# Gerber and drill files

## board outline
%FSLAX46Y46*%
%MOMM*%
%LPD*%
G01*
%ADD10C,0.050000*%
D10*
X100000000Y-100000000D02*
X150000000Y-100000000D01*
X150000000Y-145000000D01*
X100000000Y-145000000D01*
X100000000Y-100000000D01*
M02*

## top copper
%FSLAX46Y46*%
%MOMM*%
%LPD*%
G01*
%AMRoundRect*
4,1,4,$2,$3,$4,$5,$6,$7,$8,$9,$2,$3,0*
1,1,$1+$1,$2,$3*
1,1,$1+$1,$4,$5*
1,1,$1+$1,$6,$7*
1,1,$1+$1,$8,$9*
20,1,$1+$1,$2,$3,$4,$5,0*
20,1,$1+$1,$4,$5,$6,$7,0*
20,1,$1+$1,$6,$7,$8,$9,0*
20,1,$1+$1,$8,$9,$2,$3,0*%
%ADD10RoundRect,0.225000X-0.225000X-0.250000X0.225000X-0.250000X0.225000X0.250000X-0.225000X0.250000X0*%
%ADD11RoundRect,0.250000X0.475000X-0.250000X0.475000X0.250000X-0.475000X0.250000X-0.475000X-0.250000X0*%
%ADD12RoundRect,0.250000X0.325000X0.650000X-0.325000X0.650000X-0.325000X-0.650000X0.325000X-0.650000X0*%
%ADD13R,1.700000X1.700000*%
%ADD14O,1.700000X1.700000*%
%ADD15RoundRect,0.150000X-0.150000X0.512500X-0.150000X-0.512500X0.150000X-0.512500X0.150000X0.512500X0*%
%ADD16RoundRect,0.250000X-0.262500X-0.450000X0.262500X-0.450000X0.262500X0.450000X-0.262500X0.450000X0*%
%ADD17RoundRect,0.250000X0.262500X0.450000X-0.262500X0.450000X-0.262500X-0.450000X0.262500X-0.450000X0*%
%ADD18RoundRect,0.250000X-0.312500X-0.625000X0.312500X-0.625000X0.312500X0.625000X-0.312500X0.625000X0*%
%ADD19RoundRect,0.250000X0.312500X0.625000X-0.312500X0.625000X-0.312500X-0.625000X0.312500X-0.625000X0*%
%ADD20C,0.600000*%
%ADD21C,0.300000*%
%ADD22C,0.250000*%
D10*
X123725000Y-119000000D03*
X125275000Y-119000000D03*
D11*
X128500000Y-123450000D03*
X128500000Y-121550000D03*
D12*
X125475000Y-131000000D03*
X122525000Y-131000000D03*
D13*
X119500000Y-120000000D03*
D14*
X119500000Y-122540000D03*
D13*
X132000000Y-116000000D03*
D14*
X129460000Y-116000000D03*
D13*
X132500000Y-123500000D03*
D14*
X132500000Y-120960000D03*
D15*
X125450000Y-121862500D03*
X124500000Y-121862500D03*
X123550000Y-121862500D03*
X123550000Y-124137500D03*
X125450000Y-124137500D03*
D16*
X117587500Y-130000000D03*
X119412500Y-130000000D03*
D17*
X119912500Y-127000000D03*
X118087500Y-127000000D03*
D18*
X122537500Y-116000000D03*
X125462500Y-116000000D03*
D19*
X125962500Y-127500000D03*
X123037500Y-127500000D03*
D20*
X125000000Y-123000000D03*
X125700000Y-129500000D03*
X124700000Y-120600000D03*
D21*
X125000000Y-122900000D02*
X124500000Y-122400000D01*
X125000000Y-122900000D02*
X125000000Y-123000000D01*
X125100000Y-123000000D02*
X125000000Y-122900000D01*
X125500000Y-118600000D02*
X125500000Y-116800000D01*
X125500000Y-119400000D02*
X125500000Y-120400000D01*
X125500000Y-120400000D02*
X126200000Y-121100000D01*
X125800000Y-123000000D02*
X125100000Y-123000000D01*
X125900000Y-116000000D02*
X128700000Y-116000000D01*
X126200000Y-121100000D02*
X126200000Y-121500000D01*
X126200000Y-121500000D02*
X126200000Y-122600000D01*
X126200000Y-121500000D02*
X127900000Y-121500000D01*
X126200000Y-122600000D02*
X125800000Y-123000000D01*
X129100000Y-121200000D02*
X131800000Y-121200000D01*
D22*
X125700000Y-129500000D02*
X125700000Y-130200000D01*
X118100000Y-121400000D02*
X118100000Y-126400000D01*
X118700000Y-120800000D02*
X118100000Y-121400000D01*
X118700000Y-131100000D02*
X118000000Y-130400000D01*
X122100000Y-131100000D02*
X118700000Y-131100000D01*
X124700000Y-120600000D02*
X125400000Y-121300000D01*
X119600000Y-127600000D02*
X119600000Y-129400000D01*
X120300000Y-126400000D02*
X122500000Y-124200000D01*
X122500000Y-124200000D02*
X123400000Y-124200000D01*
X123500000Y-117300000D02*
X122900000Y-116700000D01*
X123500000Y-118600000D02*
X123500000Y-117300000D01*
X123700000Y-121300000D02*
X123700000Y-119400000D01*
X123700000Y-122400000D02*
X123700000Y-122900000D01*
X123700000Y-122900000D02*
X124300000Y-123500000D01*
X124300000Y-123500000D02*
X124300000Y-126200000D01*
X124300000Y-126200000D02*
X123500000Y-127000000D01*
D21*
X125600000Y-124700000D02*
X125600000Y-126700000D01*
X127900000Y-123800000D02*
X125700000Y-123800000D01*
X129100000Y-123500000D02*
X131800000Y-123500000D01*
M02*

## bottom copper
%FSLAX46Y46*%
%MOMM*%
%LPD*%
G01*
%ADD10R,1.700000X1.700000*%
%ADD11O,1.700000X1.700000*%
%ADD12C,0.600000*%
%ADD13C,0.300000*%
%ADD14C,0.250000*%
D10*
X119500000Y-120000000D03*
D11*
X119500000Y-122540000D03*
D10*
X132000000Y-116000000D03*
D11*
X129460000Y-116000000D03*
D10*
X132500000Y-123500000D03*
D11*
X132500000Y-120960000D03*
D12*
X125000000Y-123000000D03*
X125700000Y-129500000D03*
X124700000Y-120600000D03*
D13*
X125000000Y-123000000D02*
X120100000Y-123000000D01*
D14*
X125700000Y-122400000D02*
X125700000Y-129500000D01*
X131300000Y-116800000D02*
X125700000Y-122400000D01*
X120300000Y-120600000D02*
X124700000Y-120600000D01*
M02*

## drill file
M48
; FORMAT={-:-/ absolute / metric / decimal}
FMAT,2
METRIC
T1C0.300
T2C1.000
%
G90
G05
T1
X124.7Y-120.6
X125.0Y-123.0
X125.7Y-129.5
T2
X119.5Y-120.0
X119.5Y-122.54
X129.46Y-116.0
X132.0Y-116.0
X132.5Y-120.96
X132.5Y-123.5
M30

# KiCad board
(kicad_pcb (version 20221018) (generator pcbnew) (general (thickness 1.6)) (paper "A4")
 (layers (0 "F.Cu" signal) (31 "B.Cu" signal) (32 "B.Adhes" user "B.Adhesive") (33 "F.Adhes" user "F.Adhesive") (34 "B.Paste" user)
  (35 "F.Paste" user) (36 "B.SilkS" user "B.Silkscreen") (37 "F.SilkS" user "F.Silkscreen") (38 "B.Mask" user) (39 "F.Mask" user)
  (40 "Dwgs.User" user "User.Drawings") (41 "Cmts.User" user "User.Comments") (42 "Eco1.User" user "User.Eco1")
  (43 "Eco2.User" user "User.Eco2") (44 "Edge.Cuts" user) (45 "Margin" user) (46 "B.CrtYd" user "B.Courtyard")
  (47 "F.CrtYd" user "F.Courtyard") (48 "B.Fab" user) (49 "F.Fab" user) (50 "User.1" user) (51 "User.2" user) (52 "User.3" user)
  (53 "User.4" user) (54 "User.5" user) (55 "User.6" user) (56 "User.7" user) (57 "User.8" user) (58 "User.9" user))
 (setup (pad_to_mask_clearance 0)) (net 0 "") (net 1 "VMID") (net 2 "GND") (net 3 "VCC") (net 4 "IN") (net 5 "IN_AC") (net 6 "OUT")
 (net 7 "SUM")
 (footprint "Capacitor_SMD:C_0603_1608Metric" (layer "F.Cu") (at 124.5 119)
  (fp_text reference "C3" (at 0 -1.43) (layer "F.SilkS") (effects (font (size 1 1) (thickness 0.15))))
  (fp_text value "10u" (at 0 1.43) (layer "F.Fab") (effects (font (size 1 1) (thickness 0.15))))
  (pad "1" smd roundrect (at -0.775 0) (size 0.9 0.95) (layers "F.Cu" "F.Paste" "F.Mask") (roundrect_rratio 0.25) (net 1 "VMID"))
  (pad "2" smd roundrect (at 0.775 0) (size 0.9 0.95) (layers "F.Cu" "F.Paste" "F.Mask") (roundrect_rratio 0.25) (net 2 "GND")))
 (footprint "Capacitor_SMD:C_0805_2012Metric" (layer "F.Cu") (at 128.5 122.5 90)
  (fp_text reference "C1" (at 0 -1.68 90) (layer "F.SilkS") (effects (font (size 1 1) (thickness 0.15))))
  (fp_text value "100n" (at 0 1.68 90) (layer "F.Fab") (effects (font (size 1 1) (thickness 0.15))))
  (pad "1" smd roundrect (at -0.95 0 90) (size 1 1.45) (layers "F.Cu" "F.Paste" "F.Mask") (roundrect_rratio 0.25) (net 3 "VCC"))
  (pad "2" smd roundrect (at 0.95 0 90) (size 1 1.45) (layers "F.Cu" "F.Paste" "F.Mask") (roundrect_rratio 0.25) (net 2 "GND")))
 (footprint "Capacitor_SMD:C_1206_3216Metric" (layer "F.Cu") (at 124 131 180)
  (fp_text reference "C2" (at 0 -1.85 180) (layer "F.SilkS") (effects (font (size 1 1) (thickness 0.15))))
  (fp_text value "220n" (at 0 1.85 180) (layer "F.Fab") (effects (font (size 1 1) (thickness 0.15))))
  (pad "1" smd roundrect (at -1.475 0 180) (size 1.15 1.8) (layers "F.Cu" "F.Paste" "F.Mask") (roundrect_rratio 0.217391) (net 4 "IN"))
  (pad "2" smd roundrect (at 1.475 0 180) (size 1.15 1.8) (layers "F.Cu" "F.Paste" "F.Mask") (roundrect_rratio 0.217391) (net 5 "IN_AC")))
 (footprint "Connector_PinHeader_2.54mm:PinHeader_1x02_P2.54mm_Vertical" (layer "F.Cu") (at 119.5 120)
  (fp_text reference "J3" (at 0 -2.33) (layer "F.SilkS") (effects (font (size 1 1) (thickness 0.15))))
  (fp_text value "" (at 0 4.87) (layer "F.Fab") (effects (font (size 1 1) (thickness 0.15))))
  (pad "1" thru_hole rect (at 0 0) (size 1.7 1.7) (drill 1) (layers "*.Cu" "*.Mask") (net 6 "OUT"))
  (pad "2" thru_hole oval (at 0 2.54) (size 1.7 1.7) (drill 1) (layers "*.Cu" "*.Mask") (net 2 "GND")))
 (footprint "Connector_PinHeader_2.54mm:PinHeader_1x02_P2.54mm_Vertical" (layer "F.Cu") (at 132 116 -90)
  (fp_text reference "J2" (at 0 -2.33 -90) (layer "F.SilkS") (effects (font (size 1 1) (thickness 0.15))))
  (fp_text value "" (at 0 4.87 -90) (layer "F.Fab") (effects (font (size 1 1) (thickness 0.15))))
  (pad "1" thru_hole rect (at 0 0 270) (size 1.7 1.7) (drill 1) (layers "*.Cu" "*.Mask") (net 4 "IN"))
  (pad "2" thru_hole oval (at 0 2.54 270) (size 1.7 1.7) (drill 1) (layers "*.Cu" "*.Mask") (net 2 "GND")))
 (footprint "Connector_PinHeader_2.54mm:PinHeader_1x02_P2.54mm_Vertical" (layer "F.Cu") (at 132.5 123.5 180)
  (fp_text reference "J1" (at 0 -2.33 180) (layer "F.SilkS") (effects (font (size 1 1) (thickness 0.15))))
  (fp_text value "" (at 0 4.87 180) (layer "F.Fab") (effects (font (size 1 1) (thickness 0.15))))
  (pad "1" thru_hole rect (at 0 0 180) (size 1.7 1.7) (drill 1) (layers "*.Cu" "*.Mask") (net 3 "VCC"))
  (pad "2" thru_hole oval (at 0 2.54 180) (size 1.7 1.7) (drill 1) (layers "*.Cu" "*.Mask") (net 2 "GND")))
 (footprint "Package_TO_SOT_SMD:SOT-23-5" (layer "F.Cu") (at 124.5 123 -90)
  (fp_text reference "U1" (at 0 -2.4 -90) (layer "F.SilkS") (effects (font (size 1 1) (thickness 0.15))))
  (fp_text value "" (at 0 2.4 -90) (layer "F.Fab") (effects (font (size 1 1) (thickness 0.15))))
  (pad "1" smd roundrect (at -1.1375 -0.95 270) (size 1.325 0.6) (layers "F.Cu" "F.Paste" "F.Mask") (roundrect_rratio 0.25) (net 6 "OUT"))
  (pad "2" smd roundrect (at -1.1375 0 270) (size 1.325 0.6) (layers "F.Cu" "F.Paste" "F.Mask") (roundrect_rratio 0.25) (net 2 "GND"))
  (pad "3" smd roundrect (at -1.1375 0.95 270) (size 1.325 0.6) (layers "F.Cu" "F.Paste" "F.Mask") (roundrect_rratio 0.25) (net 1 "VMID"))
  (pad "4" smd roundrect (at 1.1375 0.95 270) (size 1.325 0.6) (layers "F.Cu" "F.Paste" "F.Mask") (roundrect_rratio 0.25) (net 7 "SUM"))
  (pad "5" smd roundrect (at 1.1375 -0.95 270) (size 1.325 0.6) (layers "F.Cu" "F.Paste" "F.Mask") (roundrect_rratio 0.25) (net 3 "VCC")))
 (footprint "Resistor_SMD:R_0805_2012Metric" (layer "F.Cu") (at 118.5 130)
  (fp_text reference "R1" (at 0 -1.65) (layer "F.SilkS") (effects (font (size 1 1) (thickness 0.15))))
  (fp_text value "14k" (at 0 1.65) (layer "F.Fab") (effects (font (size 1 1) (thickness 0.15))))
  (pad "1" smd roundrect (at -0.9125 0) (size 1.025 1.4) (layers "F.Cu" "F.Paste" "F.Mask") (roundrect_rratio 0.243902) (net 5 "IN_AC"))
  (pad "2" smd roundrect (at 0.9125 0) (size 1.025 1.4) (layers "F.Cu" "F.Paste" "F.Mask") (roundrect_rratio 0.243902) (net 7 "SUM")))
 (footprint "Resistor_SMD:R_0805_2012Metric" (layer "F.Cu") (at 119 127 180)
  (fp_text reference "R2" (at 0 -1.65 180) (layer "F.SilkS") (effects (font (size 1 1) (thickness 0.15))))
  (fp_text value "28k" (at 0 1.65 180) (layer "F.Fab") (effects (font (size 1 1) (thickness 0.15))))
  (pad "1" smd roundrect (at -0.9125 0 180) (size 1.025 1.4) (layers "F.Cu" "F.Paste" "F.Mask") (roundrect_rratio 0.243902) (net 7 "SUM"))
  (pad "2" smd roundrect (at 0.9125 0 180) (size 1.025 1.4) (layers "F.Cu" "F.Paste" "F.Mask") (roundrect_rratio 0.243902) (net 6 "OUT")))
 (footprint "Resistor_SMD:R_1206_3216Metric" (layer "F.Cu") (at 124 116)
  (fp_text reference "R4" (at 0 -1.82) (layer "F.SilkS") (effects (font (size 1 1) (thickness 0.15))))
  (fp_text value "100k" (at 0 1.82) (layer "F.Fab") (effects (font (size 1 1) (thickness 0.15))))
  (pad "1" smd roundrect (at -1.4625 0) (size 1.125 1.75) (layers "F.Cu" "F.Paste" "F.Mask") (roundrect_rratio 0.222222) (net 1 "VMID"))
  (pad "2" smd roundrect (at 1.4625 0) (size 1.125 1.75) (layers "F.Cu" "F.Paste" "F.Mask") (roundrect_rratio 0.222222) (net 2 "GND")))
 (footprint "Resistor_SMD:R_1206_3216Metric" (layer "F.Cu") (at 124.5 127.5 180)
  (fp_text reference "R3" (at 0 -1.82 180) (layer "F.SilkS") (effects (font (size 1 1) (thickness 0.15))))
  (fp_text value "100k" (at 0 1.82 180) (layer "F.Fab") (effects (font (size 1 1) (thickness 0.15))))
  (pad "1" smd roundrect (at -1.4625 0 180) (size 1.125 1.75) (layers "F.Cu" "F.Paste" "F.Mask") (roundrect_rratio 0.222222) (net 3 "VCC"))
  (pad "2" smd roundrect (at 1.4625 0 180) (size 1.125 1.75) (layers "F.Cu" "F.Paste" "F.Mask") (roundrect_rratio 0.222222) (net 1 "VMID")))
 (gr_rect (start 100 100) (end 150 145) (stroke (width 0.05) (type default)) (fill none) (layer "Edge.Cuts"))
 (segment (start 125 122.9) (end 124.5 122.4) (width 0.3) (layer "F.Cu") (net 2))
 (segment (start 125 122.9) (end 125 123) (width 0.3) (layer "F.Cu") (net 2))
 (segment (start 125.1 123) (end 125 122.9) (width 0.3) (layer "F.Cu") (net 2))
 (segment (start 125.5 118.6) (end 125.5 116.8) (width 0.3) (layer "F.Cu") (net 2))
 (segment (start 125.5 119.4) (end 125.5 120.4) (width 0.3) (layer "F.Cu") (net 2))
 (segment (start 125.5 120.4) (end 126.2 121.1) (width 0.3) (layer "F.Cu") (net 2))
 (segment (start 125.8 123) (end 125.1 123) (width 0.3) (layer "F.Cu") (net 2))
 (segment (start 125.9 116) (end 128.7 116) (width 0.3) (layer "F.Cu") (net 2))
 (segment (start 126.2 121.1) (end 126.2 121.5) (width 0.3) (layer "F.Cu") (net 2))
 (segment (start 126.2 121.5) (end 126.2 122.6) (width 0.3) (layer "F.Cu") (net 2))
 (segment (start 126.2 121.5) (end 127.9 121.5) (width 0.3) (layer "F.Cu") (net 2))
 (segment (start 126.2 122.6) (end 125.8 123) (width 0.3) (layer "F.Cu") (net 2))
 (segment (start 129.1 121.2) (end 131.8 121.2) (width 0.3) (layer "F.Cu") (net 2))
 (via (at 125 123) (size 0.6) (drill 0.3) (layers "F.Cu" "B.Cu") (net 2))
 (segment (start 125 123) (end 120.1 123) (width 0.3) (layer "B.Cu") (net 2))
 (segment (start 125.7 129.5) (end 125.7 130.2) (width 0.25) (layer "F.Cu") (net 4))
 (via (at 125.7 129.5) (size 0.6) (drill 0.3) (layers "F.Cu" "B.Cu") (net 4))
 (segment (start 118.1 121.4) (end 118.1 126.4) (width 0.25) (layer "F.Cu") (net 6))
 (segment (start 118.7 120.8) (end 118.1 121.4) (width 0.25) (layer "F.Cu") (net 6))
 (segment (start 118.7 131.1) (end 118 130.4) (width 0.25) (layer "F.Cu") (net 5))
 (segment (start 122.1 131.1) (end 118.7 131.1) (width 0.25) (layer "F.Cu") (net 5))
 (segment (start 124.7 120.6) (end 125.4 121.3) (width 0.25) (layer "F.Cu") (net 6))
 (segment (start 125.7 122.4) (end 125.7 129.5) (width 0.25) (layer "B.Cu") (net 4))
 (segment (start 131.3 116.8) (end 125.7 122.4) (width 0.25) (layer "B.Cu") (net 4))
 (via (at 124.7 120.6) (size 0.6) (drill 0.3) (layers "F.Cu" "B.Cu") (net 6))
 (segment (start 119.6 127.6) (end 119.6 129.4) (width 0.25) (layer "F.Cu") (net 7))
 (segment (start 120.3 120.6) (end 124.7 120.6) (width 0.25) (layer "B.Cu") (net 6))
 (segment (start 120.3 126.4) (end 122.5 124.2) (width 0.25) (layer "F.Cu") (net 7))
 (segment (start 122.5 124.2) (end 123.4 124.2) (width 0.25) (layer "F.Cu") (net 7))
 (segment (start 123.5 117.3) (end 122.9 116.7) (width 0.25) (layer "F.Cu") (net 1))
 (segment (start 123.5 118.6) (end 123.5 117.3) (width 0.25) (layer "F.Cu") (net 1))
 (segment (start 123.7 121.3) (end 123.7 119.4) (width 0.25) (layer "F.Cu") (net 1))
 (segment (start 123.7 122.4) (end 123.7 122.9) (width 0.25) (layer "F.Cu") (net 1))
 (segment (start 123.7 122.9) (end 124.3 123.5) (width 0.25) (layer "F.Cu") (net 1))
 (segment (start 124.3 123.5) (end 124.3 126.2) (width 0.25) (layer "F.Cu") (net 1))
 (segment (start 124.3 126.2) (end 123.5 127) (width 0.25) (layer "F.Cu") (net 1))
 (segment (start 125.6 124.7) (end 125.6 126.7) (width 0.3) (layer "F.Cu") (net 3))
 (segment (start 127.9 123.8) (end 125.7 123.8) (width 0.3) (layer "F.Cu") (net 3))
 (segment (start 129.1 123.5) (end 131.8 123.5) (width 0.3) (layer "F.Cu") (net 3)))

